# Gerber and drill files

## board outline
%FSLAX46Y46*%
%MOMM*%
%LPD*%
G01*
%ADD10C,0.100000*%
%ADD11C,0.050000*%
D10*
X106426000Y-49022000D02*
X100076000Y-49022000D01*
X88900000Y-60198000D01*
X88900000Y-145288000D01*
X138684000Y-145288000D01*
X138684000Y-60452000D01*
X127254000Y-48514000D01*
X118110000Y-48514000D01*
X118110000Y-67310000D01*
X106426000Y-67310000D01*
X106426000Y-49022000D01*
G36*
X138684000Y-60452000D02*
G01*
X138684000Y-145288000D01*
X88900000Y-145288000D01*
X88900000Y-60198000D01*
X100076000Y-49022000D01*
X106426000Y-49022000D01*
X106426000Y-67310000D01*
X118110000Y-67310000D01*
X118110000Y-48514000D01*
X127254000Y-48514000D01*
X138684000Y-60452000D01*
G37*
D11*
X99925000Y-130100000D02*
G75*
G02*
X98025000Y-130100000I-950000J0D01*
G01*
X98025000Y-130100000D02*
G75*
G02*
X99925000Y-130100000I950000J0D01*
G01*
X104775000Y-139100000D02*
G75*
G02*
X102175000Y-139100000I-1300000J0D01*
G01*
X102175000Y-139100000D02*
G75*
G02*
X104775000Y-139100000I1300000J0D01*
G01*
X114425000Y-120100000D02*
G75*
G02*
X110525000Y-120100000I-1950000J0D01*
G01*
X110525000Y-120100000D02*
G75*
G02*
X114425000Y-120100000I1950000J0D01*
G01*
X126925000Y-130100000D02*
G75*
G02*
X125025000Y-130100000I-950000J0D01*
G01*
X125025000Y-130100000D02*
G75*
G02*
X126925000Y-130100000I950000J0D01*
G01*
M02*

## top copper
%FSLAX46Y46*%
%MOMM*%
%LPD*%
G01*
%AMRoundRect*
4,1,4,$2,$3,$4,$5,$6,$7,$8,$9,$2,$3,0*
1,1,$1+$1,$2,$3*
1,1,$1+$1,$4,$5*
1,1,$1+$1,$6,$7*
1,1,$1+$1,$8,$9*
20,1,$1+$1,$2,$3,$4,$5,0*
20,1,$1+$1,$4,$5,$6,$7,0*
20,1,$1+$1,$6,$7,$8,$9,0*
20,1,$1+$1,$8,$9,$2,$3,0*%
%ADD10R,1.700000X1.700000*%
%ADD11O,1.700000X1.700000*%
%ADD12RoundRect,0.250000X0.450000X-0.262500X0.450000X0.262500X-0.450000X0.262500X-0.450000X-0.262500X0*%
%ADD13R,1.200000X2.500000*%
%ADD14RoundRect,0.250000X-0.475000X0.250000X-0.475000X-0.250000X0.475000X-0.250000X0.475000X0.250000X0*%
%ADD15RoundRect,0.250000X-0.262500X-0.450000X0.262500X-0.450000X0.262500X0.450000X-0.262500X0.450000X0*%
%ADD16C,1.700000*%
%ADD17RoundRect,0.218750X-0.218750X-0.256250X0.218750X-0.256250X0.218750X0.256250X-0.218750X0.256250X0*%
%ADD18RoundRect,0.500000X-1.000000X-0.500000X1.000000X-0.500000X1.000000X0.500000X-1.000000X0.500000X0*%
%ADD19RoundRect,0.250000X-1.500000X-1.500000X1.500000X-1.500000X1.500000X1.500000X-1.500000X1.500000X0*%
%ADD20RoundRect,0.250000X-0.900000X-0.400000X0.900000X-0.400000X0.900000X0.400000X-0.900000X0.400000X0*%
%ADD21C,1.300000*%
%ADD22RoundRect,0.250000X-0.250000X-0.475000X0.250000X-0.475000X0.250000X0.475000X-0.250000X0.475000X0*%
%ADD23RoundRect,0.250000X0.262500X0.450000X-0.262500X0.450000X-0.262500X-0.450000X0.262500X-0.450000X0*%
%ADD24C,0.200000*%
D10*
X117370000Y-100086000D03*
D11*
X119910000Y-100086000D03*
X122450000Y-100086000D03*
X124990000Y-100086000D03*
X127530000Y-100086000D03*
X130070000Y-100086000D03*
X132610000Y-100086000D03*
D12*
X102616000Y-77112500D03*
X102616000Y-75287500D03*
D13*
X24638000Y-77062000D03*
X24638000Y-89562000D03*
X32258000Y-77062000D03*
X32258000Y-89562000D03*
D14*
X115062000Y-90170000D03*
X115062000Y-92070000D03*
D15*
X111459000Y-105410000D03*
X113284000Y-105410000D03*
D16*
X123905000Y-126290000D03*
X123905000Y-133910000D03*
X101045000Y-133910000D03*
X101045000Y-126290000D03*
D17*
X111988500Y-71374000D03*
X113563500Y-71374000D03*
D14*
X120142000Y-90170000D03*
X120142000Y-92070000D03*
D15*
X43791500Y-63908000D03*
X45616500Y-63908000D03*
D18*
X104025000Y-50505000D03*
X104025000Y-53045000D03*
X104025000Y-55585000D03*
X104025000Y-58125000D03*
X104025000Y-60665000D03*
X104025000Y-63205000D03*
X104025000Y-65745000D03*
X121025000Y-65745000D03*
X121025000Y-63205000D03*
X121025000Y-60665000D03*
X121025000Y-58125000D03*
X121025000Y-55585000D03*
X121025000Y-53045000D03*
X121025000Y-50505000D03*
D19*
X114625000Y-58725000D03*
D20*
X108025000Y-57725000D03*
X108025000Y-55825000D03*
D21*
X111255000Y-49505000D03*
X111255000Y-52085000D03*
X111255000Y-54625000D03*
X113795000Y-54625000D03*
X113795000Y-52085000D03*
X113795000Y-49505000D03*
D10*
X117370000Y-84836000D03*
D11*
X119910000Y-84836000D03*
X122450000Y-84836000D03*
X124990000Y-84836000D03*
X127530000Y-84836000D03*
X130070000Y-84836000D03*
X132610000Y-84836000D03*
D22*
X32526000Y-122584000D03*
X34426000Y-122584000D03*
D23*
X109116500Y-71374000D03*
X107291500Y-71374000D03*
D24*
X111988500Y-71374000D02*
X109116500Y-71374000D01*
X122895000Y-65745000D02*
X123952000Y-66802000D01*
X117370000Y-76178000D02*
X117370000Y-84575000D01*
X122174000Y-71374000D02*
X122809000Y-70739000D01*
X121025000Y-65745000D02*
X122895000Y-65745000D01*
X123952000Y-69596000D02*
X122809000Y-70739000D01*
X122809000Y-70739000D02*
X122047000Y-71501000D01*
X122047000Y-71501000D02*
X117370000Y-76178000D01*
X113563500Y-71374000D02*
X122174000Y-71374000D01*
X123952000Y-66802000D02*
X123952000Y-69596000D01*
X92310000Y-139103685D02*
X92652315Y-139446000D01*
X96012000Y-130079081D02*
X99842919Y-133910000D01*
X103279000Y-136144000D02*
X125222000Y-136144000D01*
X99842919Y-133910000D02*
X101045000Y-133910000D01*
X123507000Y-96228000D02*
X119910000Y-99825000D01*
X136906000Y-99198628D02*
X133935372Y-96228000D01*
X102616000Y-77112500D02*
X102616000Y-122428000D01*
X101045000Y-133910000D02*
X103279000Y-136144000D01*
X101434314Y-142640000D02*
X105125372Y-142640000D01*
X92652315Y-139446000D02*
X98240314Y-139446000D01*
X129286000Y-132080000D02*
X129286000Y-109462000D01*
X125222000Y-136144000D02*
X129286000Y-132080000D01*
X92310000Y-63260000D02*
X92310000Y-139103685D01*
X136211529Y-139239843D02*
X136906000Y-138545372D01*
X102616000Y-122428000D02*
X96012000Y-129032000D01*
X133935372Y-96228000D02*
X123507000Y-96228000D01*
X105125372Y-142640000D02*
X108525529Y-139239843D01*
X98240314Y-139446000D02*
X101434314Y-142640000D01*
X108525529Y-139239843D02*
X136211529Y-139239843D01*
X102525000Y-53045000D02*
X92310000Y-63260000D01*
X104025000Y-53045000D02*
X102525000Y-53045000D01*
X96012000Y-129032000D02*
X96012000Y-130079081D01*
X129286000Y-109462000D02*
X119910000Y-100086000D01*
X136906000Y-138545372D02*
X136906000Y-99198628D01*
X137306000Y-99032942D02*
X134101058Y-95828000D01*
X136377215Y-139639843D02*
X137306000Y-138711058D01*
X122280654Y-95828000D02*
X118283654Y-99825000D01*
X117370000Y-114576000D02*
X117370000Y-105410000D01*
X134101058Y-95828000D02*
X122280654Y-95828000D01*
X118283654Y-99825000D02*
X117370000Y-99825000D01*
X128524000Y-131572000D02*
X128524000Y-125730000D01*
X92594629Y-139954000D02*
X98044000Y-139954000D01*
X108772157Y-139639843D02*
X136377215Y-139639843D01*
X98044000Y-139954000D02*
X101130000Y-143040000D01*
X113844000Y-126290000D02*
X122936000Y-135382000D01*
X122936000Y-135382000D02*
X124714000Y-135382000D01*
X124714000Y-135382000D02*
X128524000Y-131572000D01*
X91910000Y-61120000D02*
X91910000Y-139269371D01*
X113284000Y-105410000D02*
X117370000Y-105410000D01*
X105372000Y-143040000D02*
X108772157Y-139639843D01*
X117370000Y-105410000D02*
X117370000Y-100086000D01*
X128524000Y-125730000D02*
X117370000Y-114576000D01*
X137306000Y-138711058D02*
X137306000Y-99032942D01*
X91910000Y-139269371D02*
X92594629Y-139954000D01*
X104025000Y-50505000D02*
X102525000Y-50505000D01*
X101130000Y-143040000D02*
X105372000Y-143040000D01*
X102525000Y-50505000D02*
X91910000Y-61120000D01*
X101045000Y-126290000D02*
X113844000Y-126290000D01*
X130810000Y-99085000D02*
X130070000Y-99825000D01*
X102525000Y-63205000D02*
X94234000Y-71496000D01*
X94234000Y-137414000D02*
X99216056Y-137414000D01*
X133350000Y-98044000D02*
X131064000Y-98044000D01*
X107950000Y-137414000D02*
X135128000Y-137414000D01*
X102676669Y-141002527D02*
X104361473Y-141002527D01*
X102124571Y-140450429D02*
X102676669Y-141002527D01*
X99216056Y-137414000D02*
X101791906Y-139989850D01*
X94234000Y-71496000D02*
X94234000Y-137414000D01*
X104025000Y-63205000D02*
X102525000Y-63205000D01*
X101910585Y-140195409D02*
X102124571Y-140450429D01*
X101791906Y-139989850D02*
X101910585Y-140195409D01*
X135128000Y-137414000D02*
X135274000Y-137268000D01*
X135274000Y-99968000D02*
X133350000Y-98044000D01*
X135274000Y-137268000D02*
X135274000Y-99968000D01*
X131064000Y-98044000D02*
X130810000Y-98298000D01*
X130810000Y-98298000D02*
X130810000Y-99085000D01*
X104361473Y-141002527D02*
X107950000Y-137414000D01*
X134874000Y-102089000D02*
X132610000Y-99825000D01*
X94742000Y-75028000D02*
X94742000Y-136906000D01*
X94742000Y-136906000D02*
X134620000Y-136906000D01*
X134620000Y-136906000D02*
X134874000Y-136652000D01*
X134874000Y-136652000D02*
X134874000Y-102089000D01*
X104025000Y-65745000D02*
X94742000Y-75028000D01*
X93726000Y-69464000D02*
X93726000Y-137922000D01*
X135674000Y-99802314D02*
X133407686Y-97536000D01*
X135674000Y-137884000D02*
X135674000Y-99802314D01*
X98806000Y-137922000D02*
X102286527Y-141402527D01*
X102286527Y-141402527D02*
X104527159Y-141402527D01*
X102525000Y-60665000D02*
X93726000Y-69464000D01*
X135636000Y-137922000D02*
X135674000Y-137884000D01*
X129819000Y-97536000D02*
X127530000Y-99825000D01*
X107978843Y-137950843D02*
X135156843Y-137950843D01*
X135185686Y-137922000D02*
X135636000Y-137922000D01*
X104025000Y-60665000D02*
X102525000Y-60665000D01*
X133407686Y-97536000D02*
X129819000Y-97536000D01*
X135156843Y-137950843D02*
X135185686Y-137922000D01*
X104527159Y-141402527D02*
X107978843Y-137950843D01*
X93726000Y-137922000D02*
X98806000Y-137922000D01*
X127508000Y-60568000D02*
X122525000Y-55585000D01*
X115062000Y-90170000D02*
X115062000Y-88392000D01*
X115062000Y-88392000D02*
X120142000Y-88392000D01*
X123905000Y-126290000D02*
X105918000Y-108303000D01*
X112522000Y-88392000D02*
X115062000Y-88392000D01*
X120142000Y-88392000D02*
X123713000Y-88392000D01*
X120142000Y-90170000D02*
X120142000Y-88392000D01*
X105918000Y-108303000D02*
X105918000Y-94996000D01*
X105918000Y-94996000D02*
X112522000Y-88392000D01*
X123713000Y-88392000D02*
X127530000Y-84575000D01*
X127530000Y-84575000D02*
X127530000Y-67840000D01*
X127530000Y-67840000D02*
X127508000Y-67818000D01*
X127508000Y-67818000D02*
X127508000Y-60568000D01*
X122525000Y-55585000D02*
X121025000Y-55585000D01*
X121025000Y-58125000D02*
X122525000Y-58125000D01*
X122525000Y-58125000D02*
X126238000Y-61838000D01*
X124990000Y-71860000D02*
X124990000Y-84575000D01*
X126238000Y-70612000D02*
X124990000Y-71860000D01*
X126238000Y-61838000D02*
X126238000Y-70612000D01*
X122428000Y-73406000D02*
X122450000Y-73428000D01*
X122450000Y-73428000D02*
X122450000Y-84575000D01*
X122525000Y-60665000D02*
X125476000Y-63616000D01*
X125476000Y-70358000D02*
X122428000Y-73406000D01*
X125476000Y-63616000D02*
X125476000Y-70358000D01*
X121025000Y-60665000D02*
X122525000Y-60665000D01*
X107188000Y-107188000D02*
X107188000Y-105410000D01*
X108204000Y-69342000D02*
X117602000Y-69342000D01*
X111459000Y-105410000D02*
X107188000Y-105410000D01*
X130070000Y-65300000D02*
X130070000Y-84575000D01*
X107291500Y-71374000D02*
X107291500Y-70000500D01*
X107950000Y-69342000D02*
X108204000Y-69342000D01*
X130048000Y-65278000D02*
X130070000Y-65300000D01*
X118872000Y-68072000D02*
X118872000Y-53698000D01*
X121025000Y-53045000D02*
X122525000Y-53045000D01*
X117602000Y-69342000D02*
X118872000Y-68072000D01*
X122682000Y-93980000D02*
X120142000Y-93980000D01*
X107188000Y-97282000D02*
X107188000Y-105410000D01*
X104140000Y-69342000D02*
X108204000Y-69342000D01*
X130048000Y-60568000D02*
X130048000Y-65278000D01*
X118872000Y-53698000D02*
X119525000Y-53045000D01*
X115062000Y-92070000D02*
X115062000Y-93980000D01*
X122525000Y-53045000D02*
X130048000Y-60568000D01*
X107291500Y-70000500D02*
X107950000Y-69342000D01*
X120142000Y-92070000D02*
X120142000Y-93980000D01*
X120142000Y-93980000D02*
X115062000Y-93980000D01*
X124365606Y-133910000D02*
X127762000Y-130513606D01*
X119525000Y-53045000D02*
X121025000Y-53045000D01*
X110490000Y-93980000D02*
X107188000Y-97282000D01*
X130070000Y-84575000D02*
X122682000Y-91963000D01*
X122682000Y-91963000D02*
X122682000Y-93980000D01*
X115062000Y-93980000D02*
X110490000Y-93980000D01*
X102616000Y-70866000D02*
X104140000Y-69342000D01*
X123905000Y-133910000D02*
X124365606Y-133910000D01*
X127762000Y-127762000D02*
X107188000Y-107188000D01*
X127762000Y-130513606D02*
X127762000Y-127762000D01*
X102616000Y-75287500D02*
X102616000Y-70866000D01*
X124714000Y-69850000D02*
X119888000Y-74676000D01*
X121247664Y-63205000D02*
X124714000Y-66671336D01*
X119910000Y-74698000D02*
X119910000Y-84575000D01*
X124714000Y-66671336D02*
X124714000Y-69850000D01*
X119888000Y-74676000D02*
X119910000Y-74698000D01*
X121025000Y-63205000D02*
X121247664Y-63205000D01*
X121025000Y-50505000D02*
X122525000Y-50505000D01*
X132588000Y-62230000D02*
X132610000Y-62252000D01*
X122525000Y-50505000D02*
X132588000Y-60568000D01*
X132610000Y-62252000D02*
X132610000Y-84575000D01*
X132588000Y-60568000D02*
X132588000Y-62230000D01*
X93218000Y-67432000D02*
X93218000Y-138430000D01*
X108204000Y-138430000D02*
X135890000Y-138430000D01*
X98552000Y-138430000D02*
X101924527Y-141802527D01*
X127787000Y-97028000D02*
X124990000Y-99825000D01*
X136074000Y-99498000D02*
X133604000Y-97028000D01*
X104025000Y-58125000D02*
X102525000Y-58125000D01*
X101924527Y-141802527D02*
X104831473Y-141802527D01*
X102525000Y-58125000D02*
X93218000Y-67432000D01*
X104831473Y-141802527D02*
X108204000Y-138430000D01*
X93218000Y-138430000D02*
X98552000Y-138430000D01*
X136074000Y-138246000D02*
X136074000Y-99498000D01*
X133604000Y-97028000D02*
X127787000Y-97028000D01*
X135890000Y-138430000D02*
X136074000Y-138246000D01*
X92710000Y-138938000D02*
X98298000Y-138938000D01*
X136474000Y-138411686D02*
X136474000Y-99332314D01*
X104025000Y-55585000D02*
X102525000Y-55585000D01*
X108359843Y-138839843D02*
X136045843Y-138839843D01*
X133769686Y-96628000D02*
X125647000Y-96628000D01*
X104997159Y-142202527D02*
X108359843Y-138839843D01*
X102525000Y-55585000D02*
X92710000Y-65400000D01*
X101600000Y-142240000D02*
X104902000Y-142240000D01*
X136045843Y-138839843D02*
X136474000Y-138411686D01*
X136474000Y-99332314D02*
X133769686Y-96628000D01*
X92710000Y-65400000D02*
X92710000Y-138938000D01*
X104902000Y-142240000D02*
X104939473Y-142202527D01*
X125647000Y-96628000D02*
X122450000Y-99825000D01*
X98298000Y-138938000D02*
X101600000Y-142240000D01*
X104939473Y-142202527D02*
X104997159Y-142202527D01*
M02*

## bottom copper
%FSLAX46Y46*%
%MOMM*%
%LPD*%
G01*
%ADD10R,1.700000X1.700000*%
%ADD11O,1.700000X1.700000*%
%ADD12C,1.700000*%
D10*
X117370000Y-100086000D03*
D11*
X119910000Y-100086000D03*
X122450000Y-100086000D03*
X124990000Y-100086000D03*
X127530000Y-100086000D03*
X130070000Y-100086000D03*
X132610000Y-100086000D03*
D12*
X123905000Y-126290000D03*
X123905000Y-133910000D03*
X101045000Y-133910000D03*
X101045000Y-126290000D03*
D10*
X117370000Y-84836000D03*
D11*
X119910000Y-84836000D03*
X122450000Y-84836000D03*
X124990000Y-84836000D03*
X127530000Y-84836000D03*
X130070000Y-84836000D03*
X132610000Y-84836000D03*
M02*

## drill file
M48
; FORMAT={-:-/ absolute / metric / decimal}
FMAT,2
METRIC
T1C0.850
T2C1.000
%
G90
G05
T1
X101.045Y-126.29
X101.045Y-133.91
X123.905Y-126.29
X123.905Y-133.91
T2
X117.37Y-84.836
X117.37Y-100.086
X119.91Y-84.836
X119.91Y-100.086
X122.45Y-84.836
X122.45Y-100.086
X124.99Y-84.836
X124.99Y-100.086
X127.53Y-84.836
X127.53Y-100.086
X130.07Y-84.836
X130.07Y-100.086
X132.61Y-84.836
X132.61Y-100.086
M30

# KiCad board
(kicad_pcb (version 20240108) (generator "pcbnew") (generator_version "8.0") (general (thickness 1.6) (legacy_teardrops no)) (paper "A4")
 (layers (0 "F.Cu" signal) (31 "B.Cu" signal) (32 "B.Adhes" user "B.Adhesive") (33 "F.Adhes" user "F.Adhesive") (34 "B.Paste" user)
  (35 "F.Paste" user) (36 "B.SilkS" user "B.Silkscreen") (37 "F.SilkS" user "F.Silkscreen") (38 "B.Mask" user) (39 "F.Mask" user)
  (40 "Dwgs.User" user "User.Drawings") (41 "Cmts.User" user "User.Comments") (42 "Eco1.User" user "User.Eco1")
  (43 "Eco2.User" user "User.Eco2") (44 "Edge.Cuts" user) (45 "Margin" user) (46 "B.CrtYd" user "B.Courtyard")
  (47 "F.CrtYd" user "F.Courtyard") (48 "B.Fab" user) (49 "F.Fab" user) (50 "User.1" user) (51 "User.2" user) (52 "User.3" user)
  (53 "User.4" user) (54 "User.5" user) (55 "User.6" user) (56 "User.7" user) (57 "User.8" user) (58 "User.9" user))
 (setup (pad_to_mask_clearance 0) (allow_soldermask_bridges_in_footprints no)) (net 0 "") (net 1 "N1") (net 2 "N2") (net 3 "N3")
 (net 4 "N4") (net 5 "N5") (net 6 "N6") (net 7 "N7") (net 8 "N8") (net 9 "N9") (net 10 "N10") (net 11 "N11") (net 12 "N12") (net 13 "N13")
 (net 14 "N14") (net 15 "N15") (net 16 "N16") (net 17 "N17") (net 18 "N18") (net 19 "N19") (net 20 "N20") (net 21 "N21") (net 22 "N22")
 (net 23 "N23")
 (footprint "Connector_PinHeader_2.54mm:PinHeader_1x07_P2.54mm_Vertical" (layer "F.Cu") (at 117.37 100.086 90)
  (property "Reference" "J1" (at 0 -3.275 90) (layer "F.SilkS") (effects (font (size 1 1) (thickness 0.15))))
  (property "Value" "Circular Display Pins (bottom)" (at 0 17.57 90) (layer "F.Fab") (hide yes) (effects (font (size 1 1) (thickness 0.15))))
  (pad "1" thru_hole rect (at 0 0 90) (size 1.7 1.7) (drill 1) (layers "*.Cu" "*.Mask") (remove_unused_layers no) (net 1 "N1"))
  (pad "2" thru_hole oval (at 0 2.54 90) (size 1.7 1.7) (drill 1) (layers "*.Cu" "*.Mask") (remove_unused_layers no) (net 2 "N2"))
  (pad "3" thru_hole oval (at 0 5.08 90) (size 1.7 1.7) (drill 1) (layers "*.Cu" "*.Mask") (remove_unused_layers no) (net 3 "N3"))
  (pad "4" thru_hole oval (at 0 7.62 90) (size 1.7 1.7) (drill 1) (layers "*.Cu" "*.Mask") (remove_unused_layers no) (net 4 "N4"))
  (pad "5" thru_hole oval (at 0 10.16 90) (size 1.7 1.7) (drill 1) (layers "*.Cu" "*.Mask") (remove_unused_layers no) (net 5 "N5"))
  (pad "6" thru_hole oval (at 0 12.7 90) (size 1.7 1.7) (drill 1) (layers "*.Cu" "*.Mask") (remove_unused_layers no) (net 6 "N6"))
  (pad "7" thru_hole oval (at 0 15.24 90) (size 1.7 1.7) (drill 1) (layers "*.Cu" "*.Mask") (remove_unused_layers no) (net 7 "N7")))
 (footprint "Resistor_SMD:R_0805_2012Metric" (layer "F.Cu") (at 102.616 76.2 90)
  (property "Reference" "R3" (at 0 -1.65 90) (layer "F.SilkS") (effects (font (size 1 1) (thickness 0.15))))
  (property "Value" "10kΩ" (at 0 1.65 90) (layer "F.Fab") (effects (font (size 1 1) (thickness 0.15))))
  (pad "1" smd roundrect (at -0.9125 0 90) (size 1.025 1.4) (layers "F.Cu" "F.Paste" "F.Mask") (roundrect_rratio 0.243902) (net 2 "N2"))
  (pad "2" smd roundrect (at 0.9125 0 90) (size 1.025 1.4) (layers "F.Cu" "F.Paste" "F.Mask") (roundrect_rratio 0.243902) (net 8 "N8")))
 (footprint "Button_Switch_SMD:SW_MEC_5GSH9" (layer "F.Cu") (at 28.448 83.312)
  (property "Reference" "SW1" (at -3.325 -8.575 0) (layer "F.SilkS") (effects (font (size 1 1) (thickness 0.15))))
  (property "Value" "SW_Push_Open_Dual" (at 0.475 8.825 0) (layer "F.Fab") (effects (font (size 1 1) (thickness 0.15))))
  (pad "1" smd rect (at -3.81 -6.25 90) (size 2.5 1.2) (layers "F.Cu" "F.Paste" "F.Mask") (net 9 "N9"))
  (pad "2" smd rect (at -3.81 6.25 90) (size 2.5 1.2) (layers "F.Cu" "F.Paste" "F.Mask") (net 8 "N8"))
  (pad "3" smd rect (at 3.81 -6.25 90) (size 2.5 1.2) (layers "F.Cu" "F.Paste" "F.Mask") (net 9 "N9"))
  (pad "4" smd rect (at 3.81 6.25 90) (size 2.5 1.2) (layers "F.Cu" "F.Paste" "F.Mask") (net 8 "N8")))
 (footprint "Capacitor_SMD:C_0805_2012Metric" (layer "F.Cu") (at 115.062 91.12 -90)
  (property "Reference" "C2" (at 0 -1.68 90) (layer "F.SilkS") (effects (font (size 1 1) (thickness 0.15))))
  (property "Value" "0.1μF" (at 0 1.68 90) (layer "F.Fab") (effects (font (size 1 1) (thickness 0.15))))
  (pad "1" smd roundrect (at -0.95 0 270) (size 1 1.45) (layers "F.Cu" "F.Paste" "F.Mask") (roundrect_rratio 0.25) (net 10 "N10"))
  (pad "2" smd roundrect (at 0.95 0 270) (size 1 1.45) (layers "F.Cu" "F.Paste" "F.Mask") (roundrect_rratio 0.25) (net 8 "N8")))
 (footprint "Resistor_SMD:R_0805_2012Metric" (layer "F.Cu") (at 112.3715 105.41)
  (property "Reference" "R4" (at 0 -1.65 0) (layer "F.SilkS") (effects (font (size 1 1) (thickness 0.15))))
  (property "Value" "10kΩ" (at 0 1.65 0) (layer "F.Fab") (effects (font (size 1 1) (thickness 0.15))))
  (pad "1" smd roundrect (at -0.9125 0) (size 1.025 1.4) (layers "F.Cu" "F.Paste" "F.Mask") (roundrect_rratio 0.243902) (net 8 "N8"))
  (pad "2" smd roundrect (at 0.9125 0) (size 1.025 1.4) (layers "F.Cu" "F.Paste" "F.Mask") (roundrect_rratio 0.243902) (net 1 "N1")))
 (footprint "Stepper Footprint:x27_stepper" (layer "F.Cu") (at 115.015 140.26)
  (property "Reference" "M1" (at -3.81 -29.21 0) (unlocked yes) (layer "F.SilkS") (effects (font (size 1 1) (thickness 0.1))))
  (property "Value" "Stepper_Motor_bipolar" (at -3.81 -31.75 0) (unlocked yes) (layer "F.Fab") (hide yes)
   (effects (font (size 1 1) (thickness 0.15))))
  (fp_circle (center -16.04 -10.16) (end -15.09 -10.16) (stroke (width 0.05) (type default)) (fill none) (layer "Edge.Cuts"))
  (fp_circle (center -11.54 -1.16) (end -10.24 -1.16) (stroke (width 0.05) (type default)) (fill none) (layer "Edge.Cuts"))
  (fp_circle (center -2.54 -20.16) (end -0.59 -20.16) (stroke (width 0.05) (type default)) (fill none) (layer "Edge.Cuts"))
  (fp_circle (center 10.96 -10.16) (end 11.91 -10.16) (stroke (width 0.05) (type default)) (fill none) (layer "Edge.Cuts"))
  (pad "1" thru_hole circle (at 8.89 -13.97) (size 1.7 1.7) (drill 0.85) (layers "*.Cu" "*.Mask") (remove_unused_layers no) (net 10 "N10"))
  (pad "2" thru_hole circle (at 8.89 -6.35) (size 1.7 1.7) (drill 0.85) (layers "*.Cu" "*.Mask") (remove_unused_layers no) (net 8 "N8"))
  (pad "3" thru_hole circle (at -13.97 -6.35) (size 1.7 1.7) (drill 0.85) (layers "*.Cu" "*.Mask") (remove_unused_layers no) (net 2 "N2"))
  (pad "4" thru_hole circle (at -13.97 -13.97) (size 1.7 1.7) (drill 0.85) (layers "*.Cu" "*.Mask") (remove_unused_layers no) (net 1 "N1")))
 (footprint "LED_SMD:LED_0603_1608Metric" (layer "F.Cu") (at 112.776 71.374)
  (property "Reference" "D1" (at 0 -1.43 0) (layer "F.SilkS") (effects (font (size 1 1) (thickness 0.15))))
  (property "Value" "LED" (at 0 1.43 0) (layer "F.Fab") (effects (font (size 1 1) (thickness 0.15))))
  (pad "1" smd roundrect (at -0.7875 0) (size 0.875 0.95) (layers "F.Cu" "F.Paste" "F.Mask") (roundrect_rratio 0.25) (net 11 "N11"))
  (pad "2" smd roundrect (at 0.7875 0) (size 0.875 0.95) (layers "F.Cu" "F.Paste" "F.Mask") (roundrect_rratio 0.25) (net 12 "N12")))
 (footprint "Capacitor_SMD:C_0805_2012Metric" (layer "F.Cu") (at 120.142 91.12 -90)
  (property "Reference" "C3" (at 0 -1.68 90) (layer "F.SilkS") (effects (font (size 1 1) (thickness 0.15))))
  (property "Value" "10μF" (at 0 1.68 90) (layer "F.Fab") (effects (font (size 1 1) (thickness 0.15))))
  (pad "1" smd roundrect (at -0.95 0 270) (size 1 1.45) (layers "F.Cu" "F.Paste" "F.Mask") (roundrect_rratio 0.25) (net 10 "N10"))
  (pad "2" smd roundrect (at 0.95 0 270) (size 1 1.45) (layers "F.Cu" "F.Paste" "F.Mask") (roundrect_rratio 0.25) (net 8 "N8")))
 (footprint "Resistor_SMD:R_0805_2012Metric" (layer "F.Cu") (at 44.704 63.908)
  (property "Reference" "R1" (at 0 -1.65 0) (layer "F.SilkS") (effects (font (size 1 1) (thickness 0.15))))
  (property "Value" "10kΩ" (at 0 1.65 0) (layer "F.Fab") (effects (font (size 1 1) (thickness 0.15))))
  (pad "1" smd roundrect (at -0.9125 0) (size 1.025 1.4) (layers "F.Cu" "F.Paste" "F.Mask") (roundrect_rratio 0.243902) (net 10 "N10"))
  (pad "2" smd roundrect (at 0.9125 0) (size 1.025 1.4) (layers "F.Cu" "F.Paste" "F.Mask") (roundrect_rratio 0.243902) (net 9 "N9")))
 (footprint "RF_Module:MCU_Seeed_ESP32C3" (layer "F.Cu") (at 112.525 58.125)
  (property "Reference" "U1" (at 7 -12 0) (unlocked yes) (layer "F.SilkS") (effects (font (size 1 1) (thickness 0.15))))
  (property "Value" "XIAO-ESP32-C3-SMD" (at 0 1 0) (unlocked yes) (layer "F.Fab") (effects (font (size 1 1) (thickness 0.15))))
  (pad "" smd roundrect (at 1.1 -0.4) (size 1.5 1.5) (layers "F.Paste") (roundrect_rratio 0.1666666667))
  (pad "" smd roundrect (at 1.1 1.6) (size 1.5 1.5) (layers "F.Paste") (roundrect_rratio 0.1666666667))
  (pad "" smd roundrect (at 3.1 -0.4) (size 1.5 1.5) (layers "F.Paste") (roundrect_rratio 0.1666666667))
  (pad "" smd roundrect (at 3.1 1.6) (size 1.5 1.5) (layers "F.Paste") (roundrect_rratio 0.1666666667))
  (pad "1" smd roundrect (at -8.5 -7.62) (size 3 2) (layers "F.Cu" "F.Paste" "F.Mask") (roundrect_rratio 0.25) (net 1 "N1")
   (thermal_bridge_angle 45))
  (pad "2" smd roundrect (at -8.5 -5.08) (size 3 2) (layers "F.Cu" "F.Paste" "F.Mask") (roundrect_rratio 0.25) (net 2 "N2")
   (thermal_bridge_angle 45))
  (pad "3" smd roundrect (at -8.5 -2.54) (size 3 2) (layers "F.Cu" "F.Paste" "F.Mask") (roundrect_rratio 0.25) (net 3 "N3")
   (thermal_bridge_angle 45))
  (pad "4" smd roundrect (at -8.5 0) (size 3 2) (layers "F.Cu" "F.Paste" "F.Mask") (roundrect_rratio 0.25) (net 4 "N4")
   (thermal_bridge_angle 45))
  (pad "5" smd roundrect (at -8.5 2.54) (size 3 2) (layers "F.Cu" "F.Paste" "F.Mask") (roundrect_rratio 0.25) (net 5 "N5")
   (thermal_bridge_angle 45))
  (pad "6" smd roundrect (at -8.5 5.08) (size 3 2) (layers "F.Cu" "F.Paste" "F.Mask") (roundrect_rratio 0.25) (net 6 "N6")
   (thermal_bridge_angle 45))
  (pad "7" smd roundrect (at -8.5 7.62) (size 3 2) (layers "F.Cu" "F.Paste" "F.Mask") (roundrect_rratio 0.25) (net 7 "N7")
   (thermal_bridge_angle 45))
  (pad "8" smd roundrect (at 8.5 7.62) (size 3 2) (layers "F.Cu" "F.Paste" "F.Mask") (roundrect_rratio 0.25) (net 12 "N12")
   (thermal_bridge_angle 45))
  (pad "9" smd roundrect (at 8.5 5.08) (size 3 2) (layers "F.Cu" "F.Paste" "F.Mask") (roundrect_rratio 0.25) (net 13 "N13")
   (thermal_bridge_angle 45))
  (pad "10" smd roundrect (at 8.5 2.54) (size 3 2) (layers "F.Cu" "F.Paste" "F.Mask") (roundrect_rratio 0.25) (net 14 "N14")
   (thermal_bridge_angle 45))
  (pad "11" smd roundrect (at 8.5 0) (size 3 2) (layers "F.Cu" "F.Paste" "F.Mask") (roundrect_rratio 0.25) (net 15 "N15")
   (thermal_bridge_angle 45))
  (pad "12" smd roundrect (at 8.5 -2.54) (size 3 2) (layers "F.Cu" "F.Paste" "F.Mask") (roundrect_rratio 0.25) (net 10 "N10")
   (thermal_bridge_angle 45))
  (pad "13" smd roundrect (at 8.5 -5.08) (size 3 2) (layers "F.Cu" "F.Paste" "F.Mask") (roundrect_rratio 0.25) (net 8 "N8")
   (thermal_bridge_angle 45))
  (pad "14" smd roundrect (at 8.5 -7.62) (size 3 2) (layers "F.Cu" "F.Paste" "F.Mask") (roundrect_rratio 0.25) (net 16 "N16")
   (thermal_bridge_angle 45))
  (pad "15" smd roundrect (at 2.1 0.6) (size 3.5 3.5) (layers "F.Cu" "F.Mask") (roundrect_rratio 0.07142857143) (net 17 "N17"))
  (pad "16" smd roundrect (at -4.5 -0.4) (size 2.3 1.3) (layers "F.Cu" "F.Paste" "F.Mask") (roundrect_rratio 0.1923076923) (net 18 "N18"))
  (pad "17" smd roundrect (at -4.5 -2.3) (size 2.3 1.3) (layers "F.Cu" "F.Paste" "F.Mask") (roundrect_rratio 0.1923076923) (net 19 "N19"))
  (pad "18" smd circle (at -1.27 -8.62) (size 1.3 1.3) (layers "F.Cu" "F.Paste" "F.Mask") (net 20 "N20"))
  (pad "19" smd circle (at -1.27 -6.04) (size 1.3 1.3) (layers "F.Cu" "F.Paste" "F.Mask") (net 9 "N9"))
  (pad "20" smd circle (at -1.27 -3.5) (size 1.3 1.3) (layers "F.Cu" "F.Paste" "F.Mask") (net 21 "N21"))
  (pad "21" smd circle (at 1.27 -3.5) (size 1.3 1.3) (layers "F.Cu" "F.Paste" "F.Mask") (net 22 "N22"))
  (pad "22" smd circle (at 1.27 -6.04) (size 1.3 1.3) (layers "F.Cu" "F.Paste" "F.Mask") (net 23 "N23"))
  (pad "23" smd circle (at 1.27 -8.62) (size 1.3 1.3) (layers "F.Cu" "F.Paste" "F.Mask")))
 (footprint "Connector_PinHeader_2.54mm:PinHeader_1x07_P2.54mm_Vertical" (layer "F.Cu") (at 117.37 84.836 90)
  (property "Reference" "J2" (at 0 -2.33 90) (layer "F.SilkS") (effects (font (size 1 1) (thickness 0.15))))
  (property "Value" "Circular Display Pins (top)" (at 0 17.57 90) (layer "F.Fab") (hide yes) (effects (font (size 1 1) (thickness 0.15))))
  (pad "1" thru_hole rect (at 0 0 90) (size 1.7 1.7) (drill 1) (layers "*.Cu" "*.Mask") (remove_unused_layers no) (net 12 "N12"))
  (pad "2" thru_hole oval (at 0 2.54 90) (size 1.7 1.7) (drill 1) (layers "*.Cu" "*.Mask") (remove_unused_layers no) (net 13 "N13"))
  (pad "3" thru_hole oval (at 0 5.08 90) (size 1.7 1.7) (drill 1) (layers "*.Cu" "*.Mask") (remove_unused_layers no) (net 14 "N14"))
  (pad "4" thru_hole oval (at 0 7.62 90) (size 1.7 1.7) (drill 1) (layers "*.Cu" "*.Mask") (remove_unused_layers no) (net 15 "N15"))
  (pad "5" thru_hole oval (at 0 10.16 90) (size 1.7 1.7) (drill 1) (layers "*.Cu" "*.Mask") (remove_unused_layers no) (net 10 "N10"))
  (pad "6" thru_hole oval (at 0 12.7 90) (size 1.7 1.7) (drill 1) (layers "*.Cu" "*.Mask") (remove_unused_layers no) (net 8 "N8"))
  (pad "7" thru_hole oval (at 0 15.24 90) (size 1.7 1.7) (drill 1) (layers "*.Cu" "*.Mask") (remove_unused_layers no) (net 16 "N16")))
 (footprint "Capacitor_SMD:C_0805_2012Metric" (layer "F.Cu") (at 33.476 122.584)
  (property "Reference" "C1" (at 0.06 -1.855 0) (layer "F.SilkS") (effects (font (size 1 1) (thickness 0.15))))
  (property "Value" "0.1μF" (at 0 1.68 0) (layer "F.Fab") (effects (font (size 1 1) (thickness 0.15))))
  (pad "1" smd roundrect (at -0.95 0) (size 1 1.45) (layers "F.Cu" "F.Paste" "F.Mask") (roundrect_rratio 0.25) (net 8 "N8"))
  (pad "2" smd roundrect (at 0.95 0) (size 1 1.45) (layers "F.Cu" "F.Paste" "F.Mask") (roundrect_rratio 0.25) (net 9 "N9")))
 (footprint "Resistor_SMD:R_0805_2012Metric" (layer "F.Cu") (at 108.204 71.374 180)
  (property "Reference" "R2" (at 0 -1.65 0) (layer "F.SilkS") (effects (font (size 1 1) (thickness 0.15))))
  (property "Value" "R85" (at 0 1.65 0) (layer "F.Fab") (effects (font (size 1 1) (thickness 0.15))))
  (pad "1" smd roundrect (at -0.9125 0 180) (size 1.025 1.4) (layers "F.Cu" "F.Paste" "F.Mask") (roundrect_rratio 0.243902) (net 11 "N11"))
  (pad "2" smd roundrect (at 0.9125 0 180) (size 1.025 1.4) (layers "F.Cu" "F.Paste" "F.Mask") (roundrect_rratio 0.243902) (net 8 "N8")))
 (gr_poly
  (pts (xy 106.426 49.022) (xy 100.076 49.022) (xy 88.9 60.198) (xy 88.9 145.288) (xy 138.684 145.288) (xy 138.684 60.452)
   (xy 127.254 48.514) (xy 118.11 48.514) (xy 118.11 67.31) (xy 106.426 67.31))
  (stroke (width 0.1) (type solid)) (fill solid) (layer "Edge.Cuts"))
 (segment (start 111.9885 71.374) (end 109.1165 71.374) (width 0.2) (layer "F.Cu") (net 11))
 (segment (start 122.895 65.745) (end 123.952 66.802) (width 0.2) (layer "F.Cu") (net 12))
 (segment (start 117.37 76.178) (end 117.37 84.575) (width 0.2) (layer "F.Cu") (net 12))
 (segment (start 122.174 71.374) (end 122.809 70.739) (width 0.2) (layer "F.Cu") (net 12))
 (segment (start 121.025 65.745) (end 122.895 65.745) (width 0.2) (layer "F.Cu") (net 12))
 (segment (start 123.952 69.596) (end 122.809 70.739) (width 0.2) (layer "F.Cu") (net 12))
 (segment (start 122.809 70.739) (end 122.047 71.501) (width 0.2) (layer "F.Cu") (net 12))
 (segment (start 122.047 71.501) (end 117.37 76.178) (width 0.2) (layer "F.Cu") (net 12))
 (segment (start 113.5635 71.374) (end 122.174 71.374) (width 0.2) (layer "F.Cu") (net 12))
 (segment (start 123.952 66.802) (end 123.952 69.596) (width 0.2) (layer "F.Cu") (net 12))
 (segment (start 92.31 139.103685) (end 92.652315 139.446) (width 0.2) (layer "F.Cu") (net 2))
 (segment (start 96.012 130.079081) (end 99.842919 133.91) (width 0.2) (layer "F.Cu") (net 2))
 (segment (start 103.279 136.144) (end 125.222 136.144) (width 0.2) (layer "F.Cu") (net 2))
 (segment (start 99.842919 133.91) (end 101.045 133.91) (width 0.2) (layer "F.Cu") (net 2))
 (segment (start 123.507 96.228) (end 119.91 99.825) (width 0.2) (layer "F.Cu") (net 2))
 (segment (start 136.906 99.198628) (end 133.935372 96.228) (width 0.2) (layer "F.Cu") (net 2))
 (segment (start 102.616 77.1125) (end 102.616 122.428) (width 0.2) (layer "F.Cu") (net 2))
 (segment (start 101.045 133.91) (end 103.279 136.144) (width 0.2) (layer "F.Cu") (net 2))
 (segment (start 101.434314 142.64) (end 105.125372 142.64) (width 0.2) (layer "F.Cu") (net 2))
 (segment (start 92.652315 139.446) (end 98.240314 139.446) (width 0.2) (layer "F.Cu") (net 2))
 (segment (start 129.286 132.08) (end 129.286 109.462) (width 0.2) (layer "F.Cu") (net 2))
 (segment (start 125.222 136.144) (end 129.286 132.08) (width 0.2) (layer "F.Cu") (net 2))
 (segment (start 92.31 63.26) (end 92.31 139.103685) (width 0.2) (layer "F.Cu") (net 2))
 (segment (start 136.211529 139.239843) (end 136.906 138.545372) (width 0.2) (layer "F.Cu") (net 2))
 (segment (start 102.616 122.428) (end 96.012 129.032) (width 0.2) (layer "F.Cu") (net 2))
 (segment (start 133.935372 96.228) (end 123.507 96.228) (width 0.2) (layer "F.Cu") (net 2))
 (segment (start 105.125372 142.64) (end 108.525529 139.239843) (width 0.2) (layer "F.Cu") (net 2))
 (segment (start 98.240314 139.446) (end 101.434314 142.64) (width 0.2) (layer "F.Cu") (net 2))
 (segment (start 108.525529 139.239843) (end 136.211529 139.239843) (width 0.2) (layer "F.Cu") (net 2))
 (segment (start 102.525 53.045) (end 92.31 63.26) (width 0.2) (layer "F.Cu") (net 2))
 (segment (start 104.025 53.045) (end 102.525 53.045) (width 0.2) (layer "F.Cu") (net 2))
 (segment (start 96.012 129.032) (end 96.012 130.079081) (width 0.2) (layer "F.Cu") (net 2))
 (segment (start 129.286 109.462) (end 119.91 100.086) (width 0.2) (layer "F.Cu") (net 2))
 (segment (start 136.906 138.545372) (end 136.906 99.198628) (width 0.2) (layer "F.Cu") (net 2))
 (segment (start 137.306 99.032942) (end 134.101058 95.828) (width 0.2) (layer "F.Cu") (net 1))
 (segment (start 136.377215 139.639843) (end 137.306 138.711058) (width 0.2) (layer "F.Cu") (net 1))
 (segment (start 122.280654 95.828) (end 118.283654 99.825) (width 0.2) (layer "F.Cu") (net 1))
 (segment (start 117.37 114.576) (end 117.37 105.41) (width 0.2) (layer "F.Cu") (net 1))
 (segment (start 134.101058 95.828) (end 122.280654 95.828) (width 0.2) (layer "F.Cu") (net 1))
 (segment (start 118.283654 99.825) (end 117.37 99.825) (width 0.2) (layer "F.Cu") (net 1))
 (segment (start 128.524 131.572) (end 128.524 125.73) (width 0.2) (layer "F.Cu") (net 1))
 (segment (start 92.594629 139.954) (end 98.044 139.954) (width 0.2) (layer "F.Cu") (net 1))
 (segment (start 108.772157 139.639843) (end 136.377215 139.639843) (width 0.2) (layer "F.Cu") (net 1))
 (segment (start 98.044 139.954) (end 101.13 143.04) (width 0.2) (layer "F.Cu") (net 1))
 (segment (start 113.844 126.29) (end 122.936 135.382) (width 0.2) (layer "F.Cu") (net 1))
 (segment (start 122.936 135.382) (end 124.714 135.382) (width 0.2) (layer "F.Cu") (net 1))
 (segment (start 124.714 135.382) (end 128.524 131.572) (width 0.2) (layer "F.Cu") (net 1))
 (segment (start 91.91 61.12) (end 91.91 139.269371) (width 0.2) (layer "F.Cu") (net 1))
 (segment (start 113.284 105.41) (end 117.37 105.41) (width 0.2) (layer "F.Cu") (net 1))
 (segment (start 105.372 143.04) (end 108.772157 139.639843) (width 0.2) (layer "F.Cu") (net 1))
 (segment (start 117.37 105.41) (end 117.37 100.086) (width 0.2) (layer "F.Cu") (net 1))
 (segment (start 128.524 125.73) (end 117.37 114.576) (width 0.2) (layer "F.Cu") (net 1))
 (segment (start 137.306 138.711058) (end 137.306 99.032942) (width 0.2) (layer "F.Cu") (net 1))
 (segment (start 91.91 139.269371) (end 92.594629 139.954) (width 0.2) (layer "F.Cu") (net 1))
 (segment (start 104.025 50.505) (end 102.525 50.505) (width 0.2) (layer "F.Cu") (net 1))
 (segment (start 101.13 143.04) (end 105.372 143.04) (width 0.2) (layer "F.Cu") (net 1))
 (segment (start 102.525 50.505) (end 91.91 61.12) (width 0.2) (layer "F.Cu") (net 1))
 (segment (start 101.045 126.29) (end 113.844 126.29) (width 0.2) (layer "F.Cu") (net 1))
 (segment (start 130.81 99.085) (end 130.07 99.825) (width 0.2) (layer "F.Cu") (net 6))
 (segment (start 102.525 63.205) (end 94.234 71.496) (width 0.2) (layer "F.Cu") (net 6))
 (segment (start 94.234 137.414) (end 99.216056 137.414) (width 0.2) (layer "F.Cu") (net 6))
 (segment (start 133.35 98.044) (end 131.064 98.044) (width 0.2) (layer "F.Cu") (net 6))
 (segment (start 107.95 137.414) (end 135.128 137.414) (width 0.2) (layer "F.Cu") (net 6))
 (segment (start 102.676669 141.002527) (end 104.361473 141.002527) (width 0.2) (layer "F.Cu") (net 6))
 (segment (start 102.124571 140.450429) (end 102.676669 141.002527) (width 0.2) (layer "F.Cu") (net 6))
 (segment (start 99.216056 137.414) (end 101.791906 139.98985) (width 0.2) (layer "F.Cu") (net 6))
 (segment (start 94.234 71.496) (end 94.234 137.414) (width 0.2) (layer "F.Cu") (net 6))
 (segment (start 104.025 63.205) (end 102.525 63.205) (width 0.2) (layer "F.Cu") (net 6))
 (segment (start 101.910585 140.195409) (end 102.124571 140.450429) (width 0.2) (layer "F.Cu") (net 6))
 (segment (start 101.791906 139.98985) (end 101.910585 140.195409) (width 0.2) (layer "F.Cu") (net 6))
 (segment (start 135.128 137.414) (end 135.274 137.268) (width 0.2) (layer "F.Cu") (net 6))
 (segment (start 135.274 99.968) (end 133.35 98.044) (width 0.2) (layer "F.Cu") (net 6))
 (segment (start 135.274 137.268) (end 135.274 99.968) (width 0.2) (layer "F.Cu") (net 6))
 (segment (start 131.064 98.044) (end 130.81 98.298) (width 0.2) (layer "F.Cu") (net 6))
 (segment (start 130.81 98.298) (end 130.81 99.085) (width 0.2) (layer "F.Cu") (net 6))
 (segment (start 104.361473 141.002527) (end 107.95 137.414) (width 0.2) (layer "F.Cu") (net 6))
 (segment (start 134.874 102.089) (end 132.61 99.825) (width 0.2) (layer "F.Cu") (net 7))
 (segment (start 94.742 75.028) (end 94.742 136.906) (width 0.2) (layer "F.Cu") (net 7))
 (segment (start 94.742 136.906) (end 134.62 136.906) (width 0.2) (layer "F.Cu") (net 7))
 (segment (start 134.62 136.906) (end 134.874 136.652) (width 0.2) (layer "F.Cu") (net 7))
 (segment (start 134.874 136.652) (end 134.874 102.089) (width 0.2) (layer "F.Cu") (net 7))
 (segment (start 104.025 65.745) (end 94.742 75.028) (width 0.2) (layer "F.Cu") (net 7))
 (segment (start 93.726 69.464) (end 93.726 137.922) (width 0.2) (layer "F.Cu") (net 5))
 (segment (start 135.674 99.802314) (end 133.407686 97.536) (width 0.2) (layer "F.Cu") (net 5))
 (segment (start 135.674 137.884) (end 135.674 99.802314) (width 0.2) (layer "F.Cu") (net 5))
 (segment (start 98.806 137.922) (end 102.286527 141.402527) (width 0.2) (layer "F.Cu") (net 5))
 (segment (start 102.286527 141.402527) (end 104.527159 141.402527) (width 0.2) (layer "F.Cu") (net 5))
 (segment (start 102.525 60.665) (end 93.726 69.464) (width 0.2) (layer "F.Cu") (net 5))
 (segment (start 135.636 137.922) (end 135.674 137.884) (width 0.2) (layer "F.Cu") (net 5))
 (segment (start 129.819 97.536) (end 127.53 99.825) (width 0.2) (layer "F.Cu") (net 5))
 (segment (start 107.978843 137.950843) (end 135.156843 137.950843) (width 0.2) (layer "F.Cu") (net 5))
 (segment (start 135.185686 137.922) (end 135.636 137.922) (width 0.2) (layer "F.Cu") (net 5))
 (segment (start 104.025 60.665) (end 102.525 60.665) (width 0.2) (layer "F.Cu") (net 5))
 (segment (start 133.407686 97.536) (end 129.819 97.536) (width 0.2) (layer "F.Cu") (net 5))
 (segment (start 135.156843 137.950843) (end 135.185686 137.922) (width 0.2) (layer "F.Cu") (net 5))
 (segment (start 104.527159 141.402527) (end 107.978843 137.950843) (width 0.2) (layer "F.Cu") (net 5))
 (segment (start 93.726 137.922) (end 98.806 137.922) (width 0.2) (layer "F.Cu") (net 5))
 (segment (start 127.508 60.568) (end 122.525 55.585) (width 0.2) (layer "F.Cu") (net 10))
 (segment (start 115.062 90.17) (end 115.062 88.392) (width 0.2) (layer "F.Cu") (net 10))
 (segment (start 115.062 88.392) (end 120.142 88.392) (width 0.2) (layer "F.Cu") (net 10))
 (segment (start 123.905 126.29) (end 105.918 108.303) (width 0.2) (layer "F.Cu") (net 10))
 (segment (start 112.522 88.392) (end 115.062 88.392) (width 0.2) (layer "F.Cu") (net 10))
 (segment (start 120.142 88.392) (end 123.713 88.392) (width 0.2) (layer "F.Cu") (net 10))
 (segment (start 120.142 90.17) (end 120.142 88.392) (width 0.2) (layer "F.Cu") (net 10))
 (segment (start 105.918 108.303) (end 105.918 94.996) (width 0.2) (layer "F.Cu") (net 10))
 (segment (start 105.918 94.996) (end 112.522 88.392) (width 0.2) (layer "F.Cu") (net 10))
 (segment (start 123.713 88.392) (end 127.53 84.575) (width 0.2) (layer "F.Cu") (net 10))
 (segment (start 127.53 84.575) (end 127.53 67.84) (width 0.2) (layer "F.Cu") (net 10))
 (segment (start 127.53 67.84) (end 127.508 67.818) (width 0.2) (layer "F.Cu") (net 10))
 (segment (start 127.508 67.818) (end 127.508 60.568) (width 0.2) (layer "F.Cu") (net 10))
 (segment (start 122.525 55.585) (end 121.025 55.585) (width 0.2) (layer "F.Cu") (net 10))
 (segment (start 121.025 58.125) (end 122.525 58.125) (width 0.2) (layer "F.Cu") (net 15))
 (segment (start 122.525 58.125) (end 126.238 61.838) (width 0.2) (layer "F.Cu") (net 15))
 (segment (start 124.99 71.86) (end 124.99 84.575) (width 0.2) (layer "F.Cu") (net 15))
 (segment (start 126.238 70.612) (end 124.99 71.86) (width 0.2) (layer "F.Cu") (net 15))
 (segment (start 126.238 61.838) (end 126.238 70.612) (width 0.2) (layer "F.Cu") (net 15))
 (segment (start 122.428 73.406) (end 122.45 73.428) (width 0.2) (layer "F.Cu") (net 14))
 (segment (start 122.45 73.428) (end 122.45 84.575) (width 0.2) (layer "F.Cu") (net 14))
 (segment (start 122.525 60.665) (end 125.476 63.616) (width 0.2) (layer "F.Cu") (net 14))
 (segment (start 125.476 70.358) (end 122.428 73.406) (width 0.2) (layer "F.Cu") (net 14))
 (segment (start 125.476 63.616) (end 125.476 70.358) (width 0.2) (layer "F.Cu") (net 14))
 (segment (start 121.025 60.665) (end 122.525 60.665) (width 0.2) (layer "F.Cu") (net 14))
 (segment (start 107.188 107.188) (end 107.188 105.41) (width 0.2) (layer "F.Cu") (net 8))
 (segment (start 108.204 69.342) (end 117.602 69.342) (width 0.2) (layer "F.Cu") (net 8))
 (segment (start 111.459 105.41) (end 107.188 105.41) (width 0.2) (layer "F.Cu") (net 8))
 (segment (start 130.07 65.3) (end 130.07 84.575) (width 0.2) (layer "F.Cu") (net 8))
 (segment (start 107.2915 71.374) (end 107.2915 70.0005) (width 0.2) (layer "F.Cu") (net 8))
 (segment (start 107.95 69.342) (end 108.204 69.342) (width 0.2) (layer "F.Cu") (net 8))
 (segment (start 130.048 65.278) (end 130.07 65.3) (width 0.2) (layer "F.Cu") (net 8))
 (segment (start 118.872 68.072) (end 118.872 53.698) (width 0.2) (layer "F.Cu") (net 8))
 (segment (start 121.025 53.045) (end 122.525 53.045) (width 0.2) (layer "F.Cu") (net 8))
 (segment (start 117.602 69.342) (end 118.872 68.072) (width 0.2) (layer "F.Cu") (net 8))
 (segment (start 122.682 93.98) (end 120.142 93.98) (width 0.2) (layer "F.Cu") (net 8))
 (segment (start 107.188 97.282) (end 107.188 105.41) (width 0.2) (layer "F.Cu") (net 8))
 (segment (start 104.14 69.342) (end 108.204 69.342) (width 0.2) (layer "F.Cu") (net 8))
 (segment (start 130.048 60.568) (end 130.048 65.278) (width 0.2) (layer "F.Cu") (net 8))
 (segment (start 118.872 53.698) (end 119.525 53.045) (width 0.2) (layer "F.Cu") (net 8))
 (segment (start 115.062 92.07) (end 115.062 93.98) (width 0.2) (layer "F.Cu") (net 8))
 (segment (start 122.525 53.045) (end 130.048 60.568) (width 0.2) (layer "F.Cu") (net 8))
 (segment (start 107.2915 70.0005) (end 107.95 69.342) (width 0.2) (layer "F.Cu") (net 8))
 (segment (start 120.142 92.07) (end 120.142 93.98) (width 0.2) (layer "F.Cu") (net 8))
 (segment (start 120.142 93.98) (end 115.062 93.98) (width 0.2) (layer "F.Cu") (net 8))
 (segment (start 124.365606 133.91) (end 127.762 130.513606) (width 0.2) (layer "F.Cu") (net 8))
 (segment (start 119.525 53.045) (end 121.025 53.045) (width 0.2) (layer "F.Cu") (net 8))
 (segment (start 110.49 93.98) (end 107.188 97.282) (width 0.2) (layer "F.Cu") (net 8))
 (segment (start 130.07 84.575) (end 122.682 91.963) (width 0.2) (layer "F.Cu") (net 8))
 (segment (start 122.682 91.963) (end 122.682 93.98) (width 0.2) (layer "F.Cu") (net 8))
 (segment (start 115.062 93.98) (end 110.49 93.98) (width 0.2) (layer "F.Cu") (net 8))
 (segment (start 102.616 70.866) (end 104.14 69.342) (width 0.2) (layer "F.Cu") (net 8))
 (segment (start 123.905 133.91) (end 124.365606 133.91) (width 0.2) (layer "F.Cu") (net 8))
 (segment (start 127.762 127.762) (end 107.188 107.188) (width 0.2) (layer "F.Cu") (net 8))
 (segment (start 127.762 130.513606) (end 127.762 127.762) (width 0.2) (layer "F.Cu") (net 8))
 (segment (start 102.616 75.2875) (end 102.616 70.866) (width 0.2) (layer "F.Cu") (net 8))
 (segment (start 124.714 69.85) (end 119.888 74.676) (width 0.2) (layer "F.Cu") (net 13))
 (segment (start 121.247664 63.205) (end 124.714 66.671336) (width 0.2) (layer "F.Cu") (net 13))
 (segment (start 119.91 74.698) (end 119.91 84.575) (width 0.2) (layer "F.Cu") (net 13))
 (segment (start 124.714 66.671336) (end 124.714 69.85) (width 0.2) (layer "F.Cu") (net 13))
 (segment (start 119.888 74.676) (end 119.91 74.698) (width 0.2) (layer "F.Cu") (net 13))
 (segment (start 121.025 63.205) (end 121.247664 63.205) (width 0.2) (layer "F.Cu") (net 13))
 (segment (start 121.025 50.505) (end 122.525 50.505) (width 0.2) (layer "F.Cu") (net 16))
 (segment (start 132.588 62.23) (end 132.61 62.252) (width 0.2) (layer "F.Cu") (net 16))
 (segment (start 122.525 50.505) (end 132.588 60.568) (width 0.2) (layer "F.Cu") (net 16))
 (segment (start 132.61 62.252) (end 132.61 84.575) (width 0.2) (layer "F.Cu") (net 16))
 (segment (start 132.588 60.568) (end 132.588 62.23) (width 0.2) (layer "F.Cu") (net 16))
 (segment (start 93.218 67.432) (end 93.218 138.43) (width 0.2) (layer "F.Cu") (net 4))
 (segment (start 108.204 138.43) (end 135.89 138.43) (width 0.2) (layer "F.Cu") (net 4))
 (segment (start 98.552 138.43) (end 101.924527 141.802527) (width 0.2) (layer "F.Cu") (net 4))
 (segment (start 127.787 97.028) (end 124.99 99.825) (width 0.2) (layer "F.Cu") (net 4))
 (segment (start 136.074 99.498) (end 133.604 97.028) (width 0.2) (layer "F.Cu") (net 4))
 (segment (start 104.025 58.125) (end 102.525 58.125) (width 0.2) (layer "F.Cu") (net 4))
 (segment (start 101.924527 141.802527) (end 104.831473 141.802527) (width 0.2) (layer "F.Cu") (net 4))
 (segment (start 102.525 58.125) (end 93.218 67.432) (width 0.2) (layer "F.Cu") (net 4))
 (segment (start 104.831473 141.802527) (end 108.204 138.43) (width 0.2) (layer "F.Cu") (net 4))
 (segment (start 93.218 138.43) (end 98.552 138.43) (width 0.2) (layer "F.Cu") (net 4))
 (segment (start 136.074 138.246) (end 136.074 99.498) (width 0.2) (layer "F.Cu") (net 4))
 (segment (start 133.604 97.028) (end 127.787 97.028) (width 0.2) (layer "F.Cu") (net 4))
 (segment (start 135.89 138.43) (end 136.074 138.246) (width 0.2) (layer "F.Cu") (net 4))
 (segment (start 92.71 138.938) (end 98.298 138.938) (width 0.2) (layer "F.Cu") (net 3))
 (segment (start 136.474 138.411686) (end 136.474 99.332314) (width 0.2) (layer "F.Cu") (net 3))
 (segment (start 104.025 55.585) (end 102.525 55.585) (width 0.2) (layer "F.Cu") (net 3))
 (segment (start 108.359843 138.839843) (end 136.045843 138.839843) (width 0.2) (layer "F.Cu") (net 3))
 (segment (start 133.769686 96.628) (end 125.647 96.628) (width 0.2) (layer "F.Cu") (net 3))
 (segment (start 104.997159 142.202527) (end 108.359843 138.839843) (width 0.2) (layer "F.Cu") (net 3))
 (segment (start 102.525 55.585) (end 92.71 65.4) (width 0.2) (layer "F.Cu") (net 3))
 (segment (start 101.6 142.24) (end 104.902 142.24) (width 0.2) (layer "F.Cu") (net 3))
 (segment (start 136.045843 138.839843) (end 136.474 138.411686) (width 0.2) (layer "F.Cu") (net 3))
 (segment (start 136.474 99.332314) (end 133.769686 96.628) (width 0.2) (layer "F.Cu") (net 3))
 (segment (start 92.71 65.4) (end 92.71 138.938) (width 0.2) (layer "F.Cu") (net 3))
 (segment (start 104.902 142.24) (end 104.939473 142.202527) (width 0.2) (layer "F.Cu") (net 3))
 (segment (start 125.647 96.628) (end 122.45 99.825) (width 0.2) (layer "F.Cu") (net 3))
 (segment (start 98.298 138.938) (end 101.6 142.24) (width 0.2) (layer "F.Cu") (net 3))
 (segment (start 104.939473 142.202527) (end 104.997159 142.202527) (width 0.2) (layer "F.Cu") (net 3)))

